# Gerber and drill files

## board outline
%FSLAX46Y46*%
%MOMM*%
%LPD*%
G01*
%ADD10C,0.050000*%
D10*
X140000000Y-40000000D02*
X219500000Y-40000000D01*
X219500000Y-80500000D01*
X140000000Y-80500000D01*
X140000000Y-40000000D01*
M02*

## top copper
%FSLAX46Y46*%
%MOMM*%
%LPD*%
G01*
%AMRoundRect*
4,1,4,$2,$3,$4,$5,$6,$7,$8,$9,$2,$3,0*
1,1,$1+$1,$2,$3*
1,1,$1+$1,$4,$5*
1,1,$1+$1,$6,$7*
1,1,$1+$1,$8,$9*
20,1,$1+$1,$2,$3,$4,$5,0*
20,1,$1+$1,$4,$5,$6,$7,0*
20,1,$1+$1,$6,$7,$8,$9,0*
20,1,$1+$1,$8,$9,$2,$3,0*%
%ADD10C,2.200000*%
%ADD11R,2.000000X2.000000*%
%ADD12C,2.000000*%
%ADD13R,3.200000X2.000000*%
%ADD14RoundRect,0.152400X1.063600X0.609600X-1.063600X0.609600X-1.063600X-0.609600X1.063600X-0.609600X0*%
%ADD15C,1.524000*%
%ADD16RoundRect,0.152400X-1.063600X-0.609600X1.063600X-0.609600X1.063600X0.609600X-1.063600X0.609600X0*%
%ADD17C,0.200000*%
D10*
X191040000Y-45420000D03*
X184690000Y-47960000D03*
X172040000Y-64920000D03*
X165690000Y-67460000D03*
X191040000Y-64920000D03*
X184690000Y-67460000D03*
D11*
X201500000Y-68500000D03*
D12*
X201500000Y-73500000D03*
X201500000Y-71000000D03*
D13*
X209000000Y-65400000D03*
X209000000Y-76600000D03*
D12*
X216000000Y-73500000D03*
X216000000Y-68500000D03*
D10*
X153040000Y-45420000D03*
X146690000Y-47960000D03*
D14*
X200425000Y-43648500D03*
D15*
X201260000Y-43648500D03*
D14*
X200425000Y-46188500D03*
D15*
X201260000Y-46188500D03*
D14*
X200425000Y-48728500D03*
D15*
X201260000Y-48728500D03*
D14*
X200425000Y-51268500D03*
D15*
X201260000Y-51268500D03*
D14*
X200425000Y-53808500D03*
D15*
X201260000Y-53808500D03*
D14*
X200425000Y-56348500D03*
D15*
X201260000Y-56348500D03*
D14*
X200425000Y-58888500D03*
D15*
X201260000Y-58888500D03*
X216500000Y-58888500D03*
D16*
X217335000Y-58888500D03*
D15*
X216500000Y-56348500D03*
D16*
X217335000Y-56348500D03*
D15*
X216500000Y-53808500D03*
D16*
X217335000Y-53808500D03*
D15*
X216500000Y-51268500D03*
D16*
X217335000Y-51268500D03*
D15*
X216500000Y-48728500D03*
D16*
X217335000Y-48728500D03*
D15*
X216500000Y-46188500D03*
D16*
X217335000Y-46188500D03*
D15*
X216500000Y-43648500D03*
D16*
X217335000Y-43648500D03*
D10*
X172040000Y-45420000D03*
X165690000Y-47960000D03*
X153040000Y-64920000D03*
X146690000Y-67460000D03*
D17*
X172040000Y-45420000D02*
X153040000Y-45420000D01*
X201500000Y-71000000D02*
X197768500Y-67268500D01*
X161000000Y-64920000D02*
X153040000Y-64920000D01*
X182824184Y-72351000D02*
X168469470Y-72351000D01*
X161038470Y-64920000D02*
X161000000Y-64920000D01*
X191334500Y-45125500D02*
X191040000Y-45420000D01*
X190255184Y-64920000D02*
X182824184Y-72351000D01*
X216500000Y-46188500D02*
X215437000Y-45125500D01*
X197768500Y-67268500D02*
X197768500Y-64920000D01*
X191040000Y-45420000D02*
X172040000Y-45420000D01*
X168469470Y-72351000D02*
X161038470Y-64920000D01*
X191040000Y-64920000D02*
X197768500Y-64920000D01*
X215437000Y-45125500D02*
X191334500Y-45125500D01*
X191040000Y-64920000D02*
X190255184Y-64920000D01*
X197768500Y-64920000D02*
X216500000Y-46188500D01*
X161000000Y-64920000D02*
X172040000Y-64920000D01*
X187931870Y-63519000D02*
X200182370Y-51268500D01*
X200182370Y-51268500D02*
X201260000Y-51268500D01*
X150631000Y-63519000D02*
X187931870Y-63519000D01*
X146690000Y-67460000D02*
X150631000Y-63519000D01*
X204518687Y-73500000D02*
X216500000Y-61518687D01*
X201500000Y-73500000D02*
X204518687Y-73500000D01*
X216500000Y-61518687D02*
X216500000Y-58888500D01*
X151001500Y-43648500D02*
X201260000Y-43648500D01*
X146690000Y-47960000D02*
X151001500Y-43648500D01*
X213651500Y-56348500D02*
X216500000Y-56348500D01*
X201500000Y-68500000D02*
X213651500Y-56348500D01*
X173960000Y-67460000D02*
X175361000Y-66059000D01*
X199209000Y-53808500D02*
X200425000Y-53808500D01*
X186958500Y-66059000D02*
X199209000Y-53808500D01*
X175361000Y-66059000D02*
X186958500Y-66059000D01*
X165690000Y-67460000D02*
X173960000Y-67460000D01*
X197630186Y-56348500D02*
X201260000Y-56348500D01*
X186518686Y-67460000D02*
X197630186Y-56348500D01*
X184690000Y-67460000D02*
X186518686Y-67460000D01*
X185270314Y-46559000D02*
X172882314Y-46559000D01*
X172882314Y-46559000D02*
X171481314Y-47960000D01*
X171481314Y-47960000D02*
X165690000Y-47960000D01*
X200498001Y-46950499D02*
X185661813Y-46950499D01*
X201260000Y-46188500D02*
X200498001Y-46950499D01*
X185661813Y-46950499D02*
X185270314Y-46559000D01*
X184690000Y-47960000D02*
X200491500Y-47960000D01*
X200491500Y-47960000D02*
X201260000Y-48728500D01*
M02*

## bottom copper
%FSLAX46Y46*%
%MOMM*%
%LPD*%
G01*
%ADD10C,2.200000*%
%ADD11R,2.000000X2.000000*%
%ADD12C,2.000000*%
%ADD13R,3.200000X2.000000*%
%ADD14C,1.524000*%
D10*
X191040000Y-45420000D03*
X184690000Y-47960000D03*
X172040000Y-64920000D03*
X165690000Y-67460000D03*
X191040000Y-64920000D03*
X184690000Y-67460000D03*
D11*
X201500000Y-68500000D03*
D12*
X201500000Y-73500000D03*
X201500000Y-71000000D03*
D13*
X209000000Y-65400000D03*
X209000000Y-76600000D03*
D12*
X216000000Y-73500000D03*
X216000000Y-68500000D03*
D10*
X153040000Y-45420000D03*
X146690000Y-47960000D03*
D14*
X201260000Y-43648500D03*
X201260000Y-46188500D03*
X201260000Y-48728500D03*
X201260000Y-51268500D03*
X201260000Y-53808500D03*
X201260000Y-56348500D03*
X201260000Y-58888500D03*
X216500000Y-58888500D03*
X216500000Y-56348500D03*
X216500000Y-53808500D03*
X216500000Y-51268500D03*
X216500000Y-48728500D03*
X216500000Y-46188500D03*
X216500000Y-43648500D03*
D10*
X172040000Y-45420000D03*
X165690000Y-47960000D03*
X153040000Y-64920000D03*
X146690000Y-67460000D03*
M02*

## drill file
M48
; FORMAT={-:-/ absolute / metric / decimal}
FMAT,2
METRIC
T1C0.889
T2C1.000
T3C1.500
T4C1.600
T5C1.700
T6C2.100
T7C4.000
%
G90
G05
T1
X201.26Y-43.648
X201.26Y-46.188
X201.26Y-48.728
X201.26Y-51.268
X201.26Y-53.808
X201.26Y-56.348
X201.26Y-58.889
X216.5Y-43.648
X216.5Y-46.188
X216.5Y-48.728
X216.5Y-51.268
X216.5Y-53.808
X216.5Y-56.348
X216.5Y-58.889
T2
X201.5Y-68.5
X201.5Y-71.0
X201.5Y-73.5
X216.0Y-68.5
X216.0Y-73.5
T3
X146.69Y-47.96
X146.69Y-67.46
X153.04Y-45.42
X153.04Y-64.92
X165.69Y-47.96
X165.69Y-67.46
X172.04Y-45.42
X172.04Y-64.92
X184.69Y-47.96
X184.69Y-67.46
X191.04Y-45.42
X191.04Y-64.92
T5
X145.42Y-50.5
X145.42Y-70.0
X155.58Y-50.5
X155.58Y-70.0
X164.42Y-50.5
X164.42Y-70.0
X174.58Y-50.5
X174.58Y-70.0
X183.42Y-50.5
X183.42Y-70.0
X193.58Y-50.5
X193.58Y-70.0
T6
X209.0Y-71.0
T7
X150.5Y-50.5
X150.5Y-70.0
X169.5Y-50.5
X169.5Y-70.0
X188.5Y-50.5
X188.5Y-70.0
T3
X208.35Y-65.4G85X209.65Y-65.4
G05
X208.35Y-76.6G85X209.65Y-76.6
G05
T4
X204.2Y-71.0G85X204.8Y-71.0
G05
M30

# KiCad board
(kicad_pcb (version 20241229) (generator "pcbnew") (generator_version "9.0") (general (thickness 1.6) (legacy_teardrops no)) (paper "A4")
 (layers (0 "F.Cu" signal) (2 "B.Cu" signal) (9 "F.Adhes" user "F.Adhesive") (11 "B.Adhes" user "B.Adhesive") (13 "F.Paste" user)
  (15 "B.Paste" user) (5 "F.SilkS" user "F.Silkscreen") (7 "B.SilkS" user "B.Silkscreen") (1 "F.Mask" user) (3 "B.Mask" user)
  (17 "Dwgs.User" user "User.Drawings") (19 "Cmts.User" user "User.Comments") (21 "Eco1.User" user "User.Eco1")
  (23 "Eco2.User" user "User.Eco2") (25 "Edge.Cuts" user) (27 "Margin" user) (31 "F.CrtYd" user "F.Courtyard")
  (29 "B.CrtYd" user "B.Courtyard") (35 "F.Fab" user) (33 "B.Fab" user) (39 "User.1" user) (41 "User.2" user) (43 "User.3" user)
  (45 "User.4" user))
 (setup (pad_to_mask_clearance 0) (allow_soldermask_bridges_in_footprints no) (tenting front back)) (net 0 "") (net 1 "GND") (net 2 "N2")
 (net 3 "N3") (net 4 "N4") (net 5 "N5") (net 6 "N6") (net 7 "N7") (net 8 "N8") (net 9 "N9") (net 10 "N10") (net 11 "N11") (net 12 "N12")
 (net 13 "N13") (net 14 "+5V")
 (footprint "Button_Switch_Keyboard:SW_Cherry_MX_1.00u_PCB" (layer "F.Cu") (at 191.04 45.42)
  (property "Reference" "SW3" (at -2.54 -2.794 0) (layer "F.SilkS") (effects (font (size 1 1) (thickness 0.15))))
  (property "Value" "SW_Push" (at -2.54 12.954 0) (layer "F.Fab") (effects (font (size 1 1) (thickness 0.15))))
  (pad "" np_thru_hole circle (at -7.62 5.08) (size 1.7 1.7) (drill 1.7) (layers "*.Cu" "*.Mask"))
  (pad "" np_thru_hole circle (at -2.54 5.08) (size 4 4) (drill 4) (layers "*.Cu" "*.Mask"))
  (pad "" np_thru_hole circle (at 2.54 5.08) (size 1.7 1.7) (drill 1.7) (layers "*.Cu" "*.Mask"))
  (pad "1" thru_hole circle (at 0 0) (size 2.2 2.2) (drill 1.5) (layers "*.Cu" "*.Mask") (remove_unused_layers no) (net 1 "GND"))
  (pad "2" thru_hole circle (at -6.35 2.54) (size 2.2 2.2) (drill 1.5) (layers "*.Cu" "*.Mask") (remove_unused_layers no) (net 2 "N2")))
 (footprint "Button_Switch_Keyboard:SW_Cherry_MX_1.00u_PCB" (layer "F.Cu") (at 172.04 64.92)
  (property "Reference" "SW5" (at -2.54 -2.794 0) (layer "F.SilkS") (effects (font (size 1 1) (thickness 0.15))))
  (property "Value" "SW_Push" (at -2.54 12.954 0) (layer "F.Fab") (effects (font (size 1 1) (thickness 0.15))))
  (pad "" np_thru_hole circle (at -7.62 5.08) (size 1.7 1.7) (drill 1.7) (layers "*.Cu" "*.Mask"))
  (pad "" np_thru_hole circle (at -2.54 5.08) (size 4 4) (drill 4) (layers "*.Cu" "*.Mask"))
  (pad "" np_thru_hole circle (at 2.54 5.08) (size 1.7 1.7) (drill 1.7) (layers "*.Cu" "*.Mask"))
  (pad "1" thru_hole circle (at 0 0) (size 2.2 2.2) (drill 1.5) (layers "*.Cu" "*.Mask") (remove_unused_layers no) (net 1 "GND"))
  (pad "2" thru_hole circle (at -6.35 2.54) (size 2.2 2.2) (drill 1.5) (layers "*.Cu" "*.Mask") (remove_unused_layers no) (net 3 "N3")))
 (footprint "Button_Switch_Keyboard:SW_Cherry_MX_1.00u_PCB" (layer "F.Cu") (at 191.04 64.92)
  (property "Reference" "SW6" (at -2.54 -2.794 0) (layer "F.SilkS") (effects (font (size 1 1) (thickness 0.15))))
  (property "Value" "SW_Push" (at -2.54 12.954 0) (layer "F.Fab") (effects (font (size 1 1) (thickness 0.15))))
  (pad "" np_thru_hole circle (at -7.62 5.08) (size 1.7 1.7) (drill 1.7) (layers "*.Cu" "*.Mask"))
  (pad "" np_thru_hole circle (at -2.54 5.08) (size 4 4) (drill 4) (layers "*.Cu" "*.Mask"))
  (pad "" np_thru_hole circle (at 2.54 5.08) (size 1.7 1.7) (drill 1.7) (layers "*.Cu" "*.Mask"))
  (pad "1" thru_hole circle (at 0 0) (size 2.2 2.2) (drill 1.5) (layers "*.Cu" "*.Mask") (remove_unused_layers no) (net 1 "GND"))
  (pad "2" thru_hole circle (at -6.35 2.54) (size 2.2 2.2) (drill 1.5) (layers "*.Cu" "*.Mask") (remove_unused_layers no) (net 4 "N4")))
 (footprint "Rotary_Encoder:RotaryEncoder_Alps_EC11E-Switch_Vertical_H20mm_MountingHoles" (layer "F.Cu") (at 201.5 68.5)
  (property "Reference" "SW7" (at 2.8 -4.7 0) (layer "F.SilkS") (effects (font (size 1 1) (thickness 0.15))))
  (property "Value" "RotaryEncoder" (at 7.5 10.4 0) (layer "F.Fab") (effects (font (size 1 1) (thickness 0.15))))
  (pad "" np_thru_hole oval (at 3 2.5) (size 2.2 1.6) (drill oval 2.2 1.6) (layers "*.Mask"))
  (pad "" np_thru_hole circle (at 7.5 2.5) (size 2.1 2.1) (drill 2.1) (layers "*.Mask"))
  (pad "A" thru_hole rect (at 0 0) (size 2 2) (drill 1) (layers "*.Cu" "*.Mask") (remove_unused_layers no) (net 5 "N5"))
  (pad "B" thru_hole circle (at 0 5) (size 2 2) (drill 1) (layers "*.Cu" "*.Mask") (remove_unused_layers no) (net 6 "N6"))
  (pad "C" thru_hole circle (at 0 2.5) (size 2 2) (drill 1) (layers "*.Cu" "*.Mask") (remove_unused_layers no) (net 1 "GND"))
  (pad "MP" thru_hole rect (at 7.5 -3.1) (size 3.2 2) (drill oval 2.8 1.5) (layers "*.Cu" "*.Mask") (remove_unused_layers no))
  (pad "MP" thru_hole rect (at 7.5 8.1) (size 3.2 2) (drill oval 2.8 1.5) (layers "*.Cu" "*.Mask") (remove_unused_layers no))
  (pad "S1" thru_hole circle (at 14.5 5) (size 2 2) (drill 1) (layers "*.Cu" "*.Mask") (remove_unused_layers no))
  (pad "S2" thru_hole circle (at 14.5 0) (size 2 2) (drill 1) (layers "*.Cu" "*.Mask") (remove_unused_layers no)))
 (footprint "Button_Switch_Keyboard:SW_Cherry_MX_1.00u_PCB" (layer "F.Cu") (at 153.04 45.42)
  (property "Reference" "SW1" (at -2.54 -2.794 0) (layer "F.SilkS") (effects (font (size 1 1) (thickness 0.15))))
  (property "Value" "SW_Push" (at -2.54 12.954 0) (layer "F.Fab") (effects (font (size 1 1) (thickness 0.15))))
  (pad "" np_thru_hole circle (at -7.62 5.08) (size 1.7 1.7) (drill 1.7) (layers "*.Cu" "*.Mask"))
  (pad "" np_thru_hole circle (at -2.54 5.08) (size 4 4) (drill 4) (layers "*.Cu" "*.Mask"))
  (pad "" np_thru_hole circle (at 2.54 5.08) (size 1.7 1.7) (drill 1.7) (layers "*.Cu" "*.Mask"))
  (pad "1" thru_hole circle (at 0 0) (size 2.2 2.2) (drill 1.5) (layers "*.Cu" "*.Mask") (remove_unused_layers no) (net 1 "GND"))
  (pad "2" thru_hole circle (at -6.35 2.54) (size 2.2 2.2) (drill 1.5) (layers "*.Cu" "*.Mask") (remove_unused_layers no) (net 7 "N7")))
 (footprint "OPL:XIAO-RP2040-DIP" (layer "F.Cu") (at 208.88 51.2685)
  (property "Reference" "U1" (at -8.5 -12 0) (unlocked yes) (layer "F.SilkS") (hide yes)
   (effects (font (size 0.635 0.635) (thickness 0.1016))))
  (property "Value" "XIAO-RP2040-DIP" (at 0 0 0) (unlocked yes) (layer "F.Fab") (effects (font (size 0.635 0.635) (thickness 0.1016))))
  (pad "1" smd roundrect (at -8.455 -7.62 180) (size 2.432 1.524) (layers "F.Cu" "F.Mask") (roundrect_rratio 0.1) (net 7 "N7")
   (thermal_bridge_angle 45))
  (pad "1" thru_hole circle (at -7.62 -7.62 180) (size 1.524 1.524) (drill 0.889) (layers "*.Cu" "*.Mask") (remove_unused_layers no)
   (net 7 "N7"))
  (pad "2" smd roundrect (at -8.455 -5.08 180) (size 2.432 1.524) (layers "F.Cu" "F.Mask") (roundrect_rratio 0.1) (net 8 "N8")
   (thermal_bridge_angle 45))
  (pad "2" thru_hole circle (at -7.62 -5.08 180) (size 1.524 1.524) (drill 0.889) (layers "*.Cu" "*.Mask") (remove_unused_layers no)
   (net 8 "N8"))
  (pad "3" smd roundrect (at -8.455 -2.54 180) (size 2.432 1.524) (layers "F.Cu" "F.Mask") (roundrect_rratio 0.1) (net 2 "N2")
   (thermal_bridge_angle 45))
  (pad "3" thru_hole circle (at -7.62 -2.54 180) (size 1.524 1.524) (drill 0.889) (layers "*.Cu" "*.Mask") (remove_unused_layers no)
   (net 2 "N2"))
  (pad "4" smd roundrect (at -8.455 0 180) (size 2.432 1.524) (layers "F.Cu" "F.Mask") (roundrect_rratio 0.1) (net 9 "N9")
   (thermal_bridge_angle 45))
  (pad "4" thru_hole circle (at -7.62 0 180) (size 1.524 1.524) (drill 0.889) (layers "*.Cu" "*.Mask") (remove_unused_layers no)
   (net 9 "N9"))
  (pad "5" smd roundrect (at -8.455 2.54 180) (size 2.432 1.524) (layers "F.Cu" "F.Mask") (roundrect_rratio 0.1) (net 3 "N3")
   (thermal_bridge_angle 45))
  (pad "5" thru_hole circle (at -7.62 2.54 180) (size 1.524 1.524) (drill 0.889) (layers "*.Cu" "*.Mask") (remove_unused_layers no)
   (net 3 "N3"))
  (pad "6" smd roundrect (at -8.455 5.08 180) (size 2.432 1.524) (layers "F.Cu" "F.Mask") (roundrect_rratio 0.1) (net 4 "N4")
   (thermal_bridge_angle 45))
  (pad "6" thru_hole circle (at -7.62 5.08 180) (size 1.524 1.524) (drill 0.889) (layers "*.Cu" "*.Mask") (remove_unused_layers no)
   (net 4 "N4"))
  (pad "7" smd roundrect (at -8.455 7.62 180) (size 2.432 1.524) (layers "F.Cu" "F.Mask") (roundrect_rratio 0.1) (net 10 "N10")
   (thermal_bridge_angle 45))
  (pad "7" thru_hole circle (at -7.62 7.62 180) (size 1.524 1.524) (drill 0.889) (layers "*.Cu" "*.Mask") (remove_unused_layers no)
   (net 10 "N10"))
  (pad "8" thru_hole circle (at 7.62 7.62) (size 1.524 1.524) (drill 0.889) (layers "*.Cu" "*.Mask") (remove_unused_layers no) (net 6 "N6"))
  (pad "8" smd roundrect (at 8.455 7.62) (size 2.432 1.524) (layers "F.Cu" "F.Mask") (roundrect_rratio 0.1) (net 6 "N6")
   (thermal_bridge_angle 45))
  (pad "9" thru_hole circle (at 7.62 5.08) (size 1.524 1.524) (drill 0.889) (layers "*.Cu" "*.Mask") (remove_unused_layers no) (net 5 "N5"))
  (pad "9" smd roundrect (at 8.455 5.08) (size 2.432 1.524) (layers "F.Cu" "F.Mask") (roundrect_rratio 0.1) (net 5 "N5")
   (thermal_bridge_angle 45))
  (pad "10" thru_hole circle (at 7.62 2.54) (size 1.524 1.524) (drill 0.889) (layers "*.Cu" "*.Mask") (remove_unused_layers no)
   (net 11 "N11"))
  (pad "10" smd roundrect (at 8.455 2.54) (size 2.432 1.524) (layers "F.Cu" "F.Mask") (roundrect_rratio 0.1) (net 11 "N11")
   (thermal_bridge_angle 45))
  (pad "11" thru_hole circle (at 7.62 0) (size 1.524 1.524) (drill 0.889) (layers "*.Cu" "*.Mask") (remove_unused_layers no) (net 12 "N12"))
  (pad "11" smd roundrect (at 8.455 0) (size 2.432 1.524) (layers "F.Cu" "F.Mask") (roundrect_rratio 0.1) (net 12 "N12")
   (thermal_bridge_angle 45))
  (pad "12" thru_hole circle (at 7.62 -2.54) (size 1.524 1.524) (drill 0.889) (layers "*.Cu" "*.Mask") (remove_unused_layers no)
   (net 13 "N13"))
  (pad "12" smd roundrect (at 8.455 -2.54) (size 2.432 1.524) (layers "F.Cu" "F.Mask") (roundrect_rratio 0.1) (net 13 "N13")
   (thermal_bridge_angle 45))
  (pad "13" thru_hole circle (at 7.62 -5.08) (size 1.524 1.524) (drill 0.889) (layers "*.Cu" "*.Mask") (remove_unused_layers no)
   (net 1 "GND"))
  (pad "13" smd roundrect (at 8.455 -5.08) (size 2.432 1.524) (layers "F.Cu" "F.Mask") (roundrect_rratio 0.1) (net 1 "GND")
   (thermal_bridge_angle 45))
  (pad "14" thru_hole circle (at 7.62 -7.62) (size 1.524 1.524) (drill 0.889) (layers "*.Cu" "*.Mask") (remove_unused_layers no)
   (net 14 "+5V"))
  (pad "14" smd roundrect (at 8.455 -7.62) (size 2.432 1.524) (layers "F.Cu" "F.Mask") (roundrect_rratio 0.1) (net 14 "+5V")
   (thermal_bridge_angle 45)))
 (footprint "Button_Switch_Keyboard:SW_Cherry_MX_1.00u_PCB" (layer "F.Cu") (at 172.04 45.42)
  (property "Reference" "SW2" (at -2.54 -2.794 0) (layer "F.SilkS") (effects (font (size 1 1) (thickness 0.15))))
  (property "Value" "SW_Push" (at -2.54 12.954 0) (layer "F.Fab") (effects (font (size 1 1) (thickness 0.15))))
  (pad "" np_thru_hole circle (at -7.62 5.08) (size 1.7 1.7) (drill 1.7) (layers "*.Cu" "*.Mask"))
  (pad "" np_thru_hole circle (at -2.54 5.08) (size 4 4) (drill 4) (layers "*.Cu" "*.Mask"))
  (pad "" np_thru_hole circle (at 2.54 5.08) (size 1.7 1.7) (drill 1.7) (layers "*.Cu" "*.Mask"))
  (pad "1" thru_hole circle (at 0 0) (size 2.2 2.2) (drill 1.5) (layers "*.Cu" "*.Mask") (remove_unused_layers no) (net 1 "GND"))
  (pad "2" thru_hole circle (at -6.35 2.54) (size 2.2 2.2) (drill 1.5) (layers "*.Cu" "*.Mask") (remove_unused_layers no) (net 8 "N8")))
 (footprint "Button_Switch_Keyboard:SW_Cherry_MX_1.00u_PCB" (layer "F.Cu") (at 153.04 64.92)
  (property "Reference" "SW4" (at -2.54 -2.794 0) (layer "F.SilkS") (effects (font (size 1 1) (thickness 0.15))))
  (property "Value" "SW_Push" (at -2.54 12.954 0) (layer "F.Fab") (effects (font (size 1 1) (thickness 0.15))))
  (pad "" np_thru_hole circle (at -7.62 5.08) (size 1.7 1.7) (drill 1.7) (layers "*.Cu" "*.Mask"))
  (pad "" np_thru_hole circle (at -2.54 5.08) (size 4 4) (drill 4) (layers "*.Cu" "*.Mask"))
  (pad "" np_thru_hole circle (at 2.54 5.08) (size 1.7 1.7) (drill 1.7) (layers "*.Cu" "*.Mask"))
  (pad "1" thru_hole circle (at 0 0) (size 2.2 2.2) (drill 1.5) (layers "*.Cu" "*.Mask") (remove_unused_layers no) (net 1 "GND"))
  (pad "2" thru_hole circle (at -6.35 2.54) (size 2.2 2.2) (drill 1.5) (layers "*.Cu" "*.Mask") (remove_unused_layers no) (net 9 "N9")))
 (gr_rect (start 140 40) (end 219.5 80.5) (stroke (width 0.05) (type default)) (fill no) (layer "Edge.Cuts"))
 (segment (start 172.04 45.42) (end 153.04 45.42) (width 0.2) (layer "F.Cu") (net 1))
 (segment (start 201.5 71) (end 197.7685 67.2685) (width 0.2) (layer "F.Cu") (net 1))
 (segment (start 161 64.92) (end 153.04 64.92) (width 0.2) (layer "F.Cu") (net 1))
 (segment (start 182.824184 72.351) (end 168.46947 72.351) (width 0.2) (layer "F.Cu") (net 1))
 (segment (start 161.03847 64.92) (end 161 64.92) (width 0.2) (layer "F.Cu") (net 1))
 (segment (start 191.3345 45.1255) (end 191.04 45.42) (width 0.2) (layer "F.Cu") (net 1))
 (segment (start 190.255184 64.92) (end 182.824184 72.351) (width 0.2) (layer "F.Cu") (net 1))
 (segment (start 216.5 46.1885) (end 215.437 45.1255) (width 0.2) (layer "F.Cu") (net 1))
 (segment (start 197.7685 67.2685) (end 197.7685 64.92) (width 0.2) (layer "F.Cu") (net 1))
 (segment (start 191.04 45.42) (end 172.04 45.42) (width 0.2) (layer "F.Cu") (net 1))
 (segment (start 168.46947 72.351) (end 161.03847 64.92) (width 0.2) (layer "F.Cu") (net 1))
 (segment (start 191.04 64.92) (end 197.7685 64.92) (width 0.2) (layer "F.Cu") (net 1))
 (segment (start 215.437 45.1255) (end 191.3345 45.1255) (width 0.2) (layer "F.Cu") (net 1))
 (segment (start 191.04 64.92) (end 190.255184 64.92) (width 0.2) (layer "F.Cu") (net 1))
 (segment (start 197.7685 64.92) (end 216.5 46.1885) (width 0.2) (layer "F.Cu") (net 1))
 (segment (start 161 64.92) (end 172.04 64.92) (width 0.2) (layer "F.Cu") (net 1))
 (segment (start 187.93187 63.519) (end 200.18237 51.2685) (width 0.2) (layer "F.Cu") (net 9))
 (segment (start 200.18237 51.2685) (end 201.26 51.2685) (width 0.2) (layer "F.Cu") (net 9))
 (segment (start 150.631 63.519) (end 187.93187 63.519) (width 0.2) (layer "F.Cu") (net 9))
 (segment (start 146.69 67.46) (end 150.631 63.519) (width 0.2) (layer "F.Cu") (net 9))
 (segment (start 204.518687 73.5) (end 216.5 61.518687) (width 0.2) (layer "F.Cu") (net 6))
 (segment (start 201.5 73.5) (end 204.518687 73.5) (width 0.2) (layer "F.Cu") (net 6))
 (segment (start 216.5 61.518687) (end 216.5 58.8885) (width 0.2) (layer "F.Cu") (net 6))
 (segment (start 151.0015 43.6485) (end 201.26 43.6485) (width 0.2) (layer "F.Cu") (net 7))
 (segment (start 146.69 47.96) (end 151.0015 43.6485) (width 0.2) (layer "F.Cu") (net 7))
 (segment (start 213.6515 56.3485) (end 216.5 56.3485) (width 0.2) (layer "F.Cu") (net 5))
 (segment (start 201.5 68.5) (end 213.6515 56.3485) (width 0.2) (layer "F.Cu") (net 5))
 (segment (start 173.96 67.46) (end 175.361 66.059) (width 0.2) (layer "F.Cu") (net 3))
 (segment (start 199.209 53.8085) (end 200.425 53.8085) (width 0.2) (layer "F.Cu") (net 3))
 (segment (start 186.9585 66.059) (end 199.209 53.8085) (width 0.2) (layer "F.Cu") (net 3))
 (segment (start 175.361 66.059) (end 186.9585 66.059) (width 0.2) (layer "F.Cu") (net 3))
 (segment (start 165.69 67.46) (end 173.96 67.46) (width 0.2) (layer "F.Cu") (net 3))
 (segment (start 197.630186 56.3485) (end 201.26 56.3485) (width 0.2) (layer "F.Cu") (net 4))
 (segment (start 186.518686 67.46) (end 197.630186 56.3485) (width 0.2) (layer "F.Cu") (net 4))
 (segment (start 184.69 67.46) (end 186.518686 67.46) (width 0.2) (layer "F.Cu") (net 4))
 (segment (start 185.270314 46.559) (end 172.882314 46.559) (width 0.2) (layer "F.Cu") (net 8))
 (segment (start 172.882314 46.559) (end 171.481314 47.96) (width 0.2) (layer "F.Cu") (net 8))
 (segment (start 171.481314 47.96) (end 165.69 47.96) (width 0.2) (layer "F.Cu") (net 8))
 (segment (start 200.498001 46.950499) (end 185.661813 46.950499) (width 0.2) (layer "F.Cu") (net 8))
 (segment (start 201.26 46.1885) (end 200.498001 46.950499) (width 0.2) (layer "F.Cu") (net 8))
 (segment (start 185.661813 46.950499) (end 185.270314 46.559) (width 0.2) (layer "F.Cu") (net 8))
 (segment (start 184.69 47.96) (end 200.4915 47.96) (width 0.2) (layer "F.Cu") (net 2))
 (segment (start 200.4915 47.96) (end 201.26 48.7285) (width 0.2) (layer "F.Cu") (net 2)))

